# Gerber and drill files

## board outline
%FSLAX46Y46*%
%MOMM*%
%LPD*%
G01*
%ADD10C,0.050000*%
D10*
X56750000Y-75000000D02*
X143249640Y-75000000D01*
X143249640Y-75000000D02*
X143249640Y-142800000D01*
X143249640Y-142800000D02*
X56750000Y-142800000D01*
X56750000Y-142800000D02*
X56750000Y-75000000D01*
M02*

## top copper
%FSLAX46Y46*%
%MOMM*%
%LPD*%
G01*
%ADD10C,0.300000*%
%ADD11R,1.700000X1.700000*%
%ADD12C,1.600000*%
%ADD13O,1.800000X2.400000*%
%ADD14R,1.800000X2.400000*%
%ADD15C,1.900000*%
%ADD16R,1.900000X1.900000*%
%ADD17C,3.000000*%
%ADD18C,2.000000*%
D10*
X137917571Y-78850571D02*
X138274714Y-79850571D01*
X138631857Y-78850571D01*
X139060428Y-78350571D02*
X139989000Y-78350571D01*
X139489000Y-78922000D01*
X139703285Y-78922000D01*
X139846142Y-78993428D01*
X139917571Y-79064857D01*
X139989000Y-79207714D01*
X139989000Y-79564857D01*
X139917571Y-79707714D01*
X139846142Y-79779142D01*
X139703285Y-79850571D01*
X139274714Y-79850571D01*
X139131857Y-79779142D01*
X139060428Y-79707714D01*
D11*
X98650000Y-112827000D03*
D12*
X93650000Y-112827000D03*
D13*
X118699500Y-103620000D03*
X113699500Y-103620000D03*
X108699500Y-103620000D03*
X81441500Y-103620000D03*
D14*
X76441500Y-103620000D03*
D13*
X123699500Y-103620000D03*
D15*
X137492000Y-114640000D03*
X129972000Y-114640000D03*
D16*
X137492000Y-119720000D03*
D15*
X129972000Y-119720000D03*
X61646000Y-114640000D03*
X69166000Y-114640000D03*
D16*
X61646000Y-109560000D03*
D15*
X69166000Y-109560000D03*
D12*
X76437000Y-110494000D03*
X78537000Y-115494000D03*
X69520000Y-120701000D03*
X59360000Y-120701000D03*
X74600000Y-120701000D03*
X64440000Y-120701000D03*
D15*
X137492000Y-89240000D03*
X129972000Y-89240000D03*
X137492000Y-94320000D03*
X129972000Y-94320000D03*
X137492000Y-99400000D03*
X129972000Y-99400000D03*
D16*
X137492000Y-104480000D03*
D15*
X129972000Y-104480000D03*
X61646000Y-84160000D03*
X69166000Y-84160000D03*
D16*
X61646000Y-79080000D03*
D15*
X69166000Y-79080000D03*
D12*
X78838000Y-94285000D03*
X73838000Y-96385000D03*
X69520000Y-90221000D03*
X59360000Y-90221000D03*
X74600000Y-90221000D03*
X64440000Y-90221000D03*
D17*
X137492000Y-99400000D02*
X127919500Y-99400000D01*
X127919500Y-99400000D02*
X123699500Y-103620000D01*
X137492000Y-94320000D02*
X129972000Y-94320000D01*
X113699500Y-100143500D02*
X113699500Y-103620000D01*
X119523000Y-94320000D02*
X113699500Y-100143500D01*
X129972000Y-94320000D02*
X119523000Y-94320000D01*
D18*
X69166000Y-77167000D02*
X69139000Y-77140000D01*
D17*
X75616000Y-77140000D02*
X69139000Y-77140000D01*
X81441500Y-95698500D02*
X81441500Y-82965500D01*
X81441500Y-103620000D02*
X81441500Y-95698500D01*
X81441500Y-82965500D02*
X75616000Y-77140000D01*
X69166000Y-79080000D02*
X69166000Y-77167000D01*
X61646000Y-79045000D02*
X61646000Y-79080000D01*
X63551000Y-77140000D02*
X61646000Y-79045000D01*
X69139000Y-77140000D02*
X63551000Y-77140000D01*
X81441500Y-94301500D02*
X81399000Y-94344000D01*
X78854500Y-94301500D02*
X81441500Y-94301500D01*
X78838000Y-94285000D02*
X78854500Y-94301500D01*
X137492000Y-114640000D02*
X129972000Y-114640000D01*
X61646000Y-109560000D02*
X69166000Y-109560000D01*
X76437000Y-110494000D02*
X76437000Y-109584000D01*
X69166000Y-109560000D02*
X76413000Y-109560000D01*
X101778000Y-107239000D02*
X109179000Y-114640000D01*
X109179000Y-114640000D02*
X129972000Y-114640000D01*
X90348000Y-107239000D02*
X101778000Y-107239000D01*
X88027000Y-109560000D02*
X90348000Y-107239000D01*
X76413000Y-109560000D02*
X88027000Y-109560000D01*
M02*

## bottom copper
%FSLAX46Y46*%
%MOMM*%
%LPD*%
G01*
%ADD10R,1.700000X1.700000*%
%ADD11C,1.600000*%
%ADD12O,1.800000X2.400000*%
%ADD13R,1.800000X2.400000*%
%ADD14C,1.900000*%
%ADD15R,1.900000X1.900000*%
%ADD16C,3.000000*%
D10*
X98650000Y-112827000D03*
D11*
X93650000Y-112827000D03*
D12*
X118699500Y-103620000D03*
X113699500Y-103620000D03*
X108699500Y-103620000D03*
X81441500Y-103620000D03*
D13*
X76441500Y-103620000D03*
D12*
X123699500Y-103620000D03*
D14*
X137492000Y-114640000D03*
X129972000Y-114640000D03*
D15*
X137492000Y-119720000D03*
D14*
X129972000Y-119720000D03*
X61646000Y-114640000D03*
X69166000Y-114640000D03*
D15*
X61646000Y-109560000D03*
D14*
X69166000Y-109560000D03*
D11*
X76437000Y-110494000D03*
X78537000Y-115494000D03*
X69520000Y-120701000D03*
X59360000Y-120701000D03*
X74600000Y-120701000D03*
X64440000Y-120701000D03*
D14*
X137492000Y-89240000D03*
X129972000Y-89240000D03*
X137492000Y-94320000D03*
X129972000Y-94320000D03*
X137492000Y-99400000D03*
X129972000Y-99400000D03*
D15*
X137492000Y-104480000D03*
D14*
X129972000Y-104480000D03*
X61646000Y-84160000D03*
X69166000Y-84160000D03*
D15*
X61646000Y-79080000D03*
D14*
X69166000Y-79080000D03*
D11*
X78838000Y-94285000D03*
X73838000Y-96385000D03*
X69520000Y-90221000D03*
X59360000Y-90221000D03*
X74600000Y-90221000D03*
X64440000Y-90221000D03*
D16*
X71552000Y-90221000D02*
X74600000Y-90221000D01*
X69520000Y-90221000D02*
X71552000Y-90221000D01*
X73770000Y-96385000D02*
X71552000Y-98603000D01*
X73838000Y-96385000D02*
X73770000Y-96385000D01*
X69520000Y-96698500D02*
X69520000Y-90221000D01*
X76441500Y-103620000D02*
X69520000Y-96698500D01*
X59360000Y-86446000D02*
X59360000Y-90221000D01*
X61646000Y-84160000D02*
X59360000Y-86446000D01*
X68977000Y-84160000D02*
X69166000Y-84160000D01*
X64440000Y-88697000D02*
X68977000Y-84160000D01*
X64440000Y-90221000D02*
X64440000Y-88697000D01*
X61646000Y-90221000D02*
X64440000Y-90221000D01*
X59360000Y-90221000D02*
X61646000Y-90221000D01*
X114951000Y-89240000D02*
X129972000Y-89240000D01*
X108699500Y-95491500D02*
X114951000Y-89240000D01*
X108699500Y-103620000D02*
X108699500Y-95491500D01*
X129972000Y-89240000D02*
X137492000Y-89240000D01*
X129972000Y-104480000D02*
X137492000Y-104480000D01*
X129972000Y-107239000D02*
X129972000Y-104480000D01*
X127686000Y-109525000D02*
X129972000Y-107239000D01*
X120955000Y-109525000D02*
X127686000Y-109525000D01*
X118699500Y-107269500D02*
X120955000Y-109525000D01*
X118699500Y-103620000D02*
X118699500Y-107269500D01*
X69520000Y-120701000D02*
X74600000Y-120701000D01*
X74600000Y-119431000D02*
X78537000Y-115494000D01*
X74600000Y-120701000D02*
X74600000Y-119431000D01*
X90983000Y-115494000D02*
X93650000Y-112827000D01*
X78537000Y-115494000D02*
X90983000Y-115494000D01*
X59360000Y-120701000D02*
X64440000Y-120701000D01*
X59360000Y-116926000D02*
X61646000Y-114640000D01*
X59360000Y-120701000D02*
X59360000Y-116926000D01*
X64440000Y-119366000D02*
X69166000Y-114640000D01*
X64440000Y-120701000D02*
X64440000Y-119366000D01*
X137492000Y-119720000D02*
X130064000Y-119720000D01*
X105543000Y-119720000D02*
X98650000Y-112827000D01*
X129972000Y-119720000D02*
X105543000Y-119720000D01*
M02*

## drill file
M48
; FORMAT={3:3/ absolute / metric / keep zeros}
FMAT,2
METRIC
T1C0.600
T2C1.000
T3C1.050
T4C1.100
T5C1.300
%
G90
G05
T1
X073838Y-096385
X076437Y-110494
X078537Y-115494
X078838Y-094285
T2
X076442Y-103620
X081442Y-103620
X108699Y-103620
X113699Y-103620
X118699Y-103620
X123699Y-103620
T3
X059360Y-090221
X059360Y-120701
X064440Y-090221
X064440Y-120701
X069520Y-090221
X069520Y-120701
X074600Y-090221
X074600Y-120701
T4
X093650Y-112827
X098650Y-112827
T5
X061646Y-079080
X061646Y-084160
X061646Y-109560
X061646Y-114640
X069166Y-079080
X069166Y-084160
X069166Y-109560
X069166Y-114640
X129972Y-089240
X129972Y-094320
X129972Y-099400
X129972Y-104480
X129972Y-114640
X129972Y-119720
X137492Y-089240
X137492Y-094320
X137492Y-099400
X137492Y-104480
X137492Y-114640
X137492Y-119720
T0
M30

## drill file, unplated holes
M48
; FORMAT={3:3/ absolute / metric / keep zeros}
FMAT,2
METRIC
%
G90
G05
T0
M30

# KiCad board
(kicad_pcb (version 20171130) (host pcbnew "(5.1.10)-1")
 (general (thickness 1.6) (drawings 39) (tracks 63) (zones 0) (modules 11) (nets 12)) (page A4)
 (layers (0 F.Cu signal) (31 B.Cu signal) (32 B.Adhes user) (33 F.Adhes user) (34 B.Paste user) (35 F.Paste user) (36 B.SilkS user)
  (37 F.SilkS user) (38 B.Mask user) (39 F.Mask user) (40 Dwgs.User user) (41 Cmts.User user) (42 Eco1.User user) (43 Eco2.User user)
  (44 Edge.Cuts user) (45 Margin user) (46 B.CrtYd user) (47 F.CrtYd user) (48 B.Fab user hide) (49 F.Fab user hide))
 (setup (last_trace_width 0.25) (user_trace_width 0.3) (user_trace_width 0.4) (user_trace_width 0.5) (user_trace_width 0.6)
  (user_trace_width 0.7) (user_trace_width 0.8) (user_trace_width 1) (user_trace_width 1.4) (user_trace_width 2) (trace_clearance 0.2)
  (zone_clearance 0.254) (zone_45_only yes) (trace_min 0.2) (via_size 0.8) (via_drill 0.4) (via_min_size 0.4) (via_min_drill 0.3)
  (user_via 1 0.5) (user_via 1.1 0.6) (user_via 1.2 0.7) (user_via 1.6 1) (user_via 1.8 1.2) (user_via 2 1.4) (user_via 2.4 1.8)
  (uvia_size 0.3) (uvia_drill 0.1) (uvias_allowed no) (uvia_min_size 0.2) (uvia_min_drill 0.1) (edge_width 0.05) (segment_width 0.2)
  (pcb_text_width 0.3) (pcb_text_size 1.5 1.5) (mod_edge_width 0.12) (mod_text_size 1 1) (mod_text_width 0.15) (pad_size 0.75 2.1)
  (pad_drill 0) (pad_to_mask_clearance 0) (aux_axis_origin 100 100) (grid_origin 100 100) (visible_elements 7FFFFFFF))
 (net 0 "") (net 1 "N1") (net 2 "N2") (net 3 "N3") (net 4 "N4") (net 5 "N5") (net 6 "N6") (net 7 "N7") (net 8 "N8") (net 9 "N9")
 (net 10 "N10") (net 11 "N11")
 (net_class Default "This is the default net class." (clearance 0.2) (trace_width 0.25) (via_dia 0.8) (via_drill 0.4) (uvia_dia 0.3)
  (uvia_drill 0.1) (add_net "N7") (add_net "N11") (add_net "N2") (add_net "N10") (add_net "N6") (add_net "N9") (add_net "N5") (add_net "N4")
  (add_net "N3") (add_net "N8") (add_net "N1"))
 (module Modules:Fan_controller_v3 (layer F.Cu) (at 100 120.477 180)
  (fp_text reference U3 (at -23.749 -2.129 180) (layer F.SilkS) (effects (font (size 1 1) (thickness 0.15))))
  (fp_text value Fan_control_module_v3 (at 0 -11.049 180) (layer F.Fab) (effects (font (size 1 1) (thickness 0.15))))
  (pad 1 thru_hole rect (at 1.35 7.65) (size 1.7 1.7) (drill 1.1) (layers *.Cu *.Mask) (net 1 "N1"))
  (pad 2 thru_hole circle (at 6.35 7.65) (size 1.6 1.6) (drill 1.1) (layers *.Cu *.Mask) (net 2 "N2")))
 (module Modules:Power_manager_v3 (layer F.Cu) (at 100 96)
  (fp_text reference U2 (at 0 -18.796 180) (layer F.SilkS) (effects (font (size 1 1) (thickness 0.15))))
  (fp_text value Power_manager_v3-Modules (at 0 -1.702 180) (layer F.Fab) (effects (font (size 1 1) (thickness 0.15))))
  (pad 5 thru_hole oval (at 18.6995 7.62 180) (size 1.8 2.4) (drill 1) (layers *.Cu *.Mask) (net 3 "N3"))
  (pad 4 thru_hole oval (at 13.6995 7.62 180) (size 1.8 2.4) (drill 1) (layers *.Cu *.Mask) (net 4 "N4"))
  (pad 3 thru_hole oval (at 8.6995 7.62 180) (size 1.8 2.4) (drill 1) (layers *.Cu *.Mask) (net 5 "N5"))
  (pad 2 thru_hole oval (at -18.5585 7.62 180) (size 1.8 2.4) (drill 1) (layers *.Cu *.Mask) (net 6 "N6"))
  (pad 1 thru_hole rect (at -23.5585 7.62 180) (size 1.8 2.4) (drill 1) (layers *.Cu *.Mask) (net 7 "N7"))
  (pad 6 thru_hole oval (at 23.6995 7.62 180) (size 1.8 2.4) (drill 1) (layers *.Cu *.Mask) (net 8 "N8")))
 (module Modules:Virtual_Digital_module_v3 (layer F.Cu) (at 100 100)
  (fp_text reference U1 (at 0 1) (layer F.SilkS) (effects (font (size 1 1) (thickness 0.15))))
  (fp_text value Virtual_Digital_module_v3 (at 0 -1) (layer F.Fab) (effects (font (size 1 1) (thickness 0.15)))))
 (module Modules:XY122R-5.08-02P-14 (layer F.Cu) (at 137.542 119.72 90)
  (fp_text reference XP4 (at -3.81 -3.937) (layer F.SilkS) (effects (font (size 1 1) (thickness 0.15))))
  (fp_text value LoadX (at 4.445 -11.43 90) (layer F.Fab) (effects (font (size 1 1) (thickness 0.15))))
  (pad 2 thru_hole circle (at 5.08 -0.05 90) (size 1.9 1.9) (drill 1.3) (layers *.Cu *.Mask) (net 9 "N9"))
  (pad 2 thru_hole circle (at 5.08 -7.57 90) (size 1.9 1.9) (drill 1.3) (layers *.Cu *.Mask) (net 9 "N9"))
  (pad 1 thru_hole rect (at 0 -0.05 90) (size 1.9 1.9) (drill 1.3) (layers *.Cu *.Mask) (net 1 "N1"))
  (pad 1 thru_hole circle (at 0 -7.57 90) (size 1.9 1.9) (drill 1.3) (layers *.Cu *.Mask) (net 1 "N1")))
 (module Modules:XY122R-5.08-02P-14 (layer F.Cu) (at 61.596 109.56 270)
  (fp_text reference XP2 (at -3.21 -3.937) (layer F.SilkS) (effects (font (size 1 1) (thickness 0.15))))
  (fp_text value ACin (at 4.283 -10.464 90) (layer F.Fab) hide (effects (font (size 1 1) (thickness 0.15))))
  (pad 2 thru_hole circle (at 5.08 -0.05 270) (size 1.9 1.9) (drill 1.3) (layers *.Cu *.Mask) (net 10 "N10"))
  (pad 2 thru_hole circle (at 5.08 -7.57 270) (size 1.9 1.9) (drill 1.3) (layers *.Cu *.Mask) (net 10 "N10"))
  (pad 1 thru_hole rect (at 0 -0.05 270) (size 1.9 1.9) (drill 1.3) (layers *.Cu *.Mask) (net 9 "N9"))
  (pad 1 thru_hole circle (at 0 -7.57 270) (size 1.9 1.9) (drill 1.3) (layers *.Cu *.Mask) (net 9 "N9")))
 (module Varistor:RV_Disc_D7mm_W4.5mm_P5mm (layer B.Cu) (at 78.537 115.494 90)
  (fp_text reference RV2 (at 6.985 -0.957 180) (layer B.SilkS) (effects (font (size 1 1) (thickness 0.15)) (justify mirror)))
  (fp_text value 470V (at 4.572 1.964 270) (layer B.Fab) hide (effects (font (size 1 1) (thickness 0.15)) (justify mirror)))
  (pad 2 thru_hole circle (at 5 -2.1 90) (size 1.6 1.6) (drill 0.6) (layers *.Cu *.Mask) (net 9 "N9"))
  (pad 1 thru_hole circle (at 0 0 90) (size 1.6 1.6) (drill 0.6) (layers *.Cu *.Mask) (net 2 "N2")))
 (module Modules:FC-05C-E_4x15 (layer B.Cu) (at 74.6 120.701 180)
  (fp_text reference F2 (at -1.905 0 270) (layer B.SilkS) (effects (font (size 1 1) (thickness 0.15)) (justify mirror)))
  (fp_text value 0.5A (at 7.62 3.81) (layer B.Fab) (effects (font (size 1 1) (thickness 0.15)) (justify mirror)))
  (pad 1 thru_hole circle (at 5.08 0 180) (size 1.6 1.6) (drill 1.05) (layers *.Cu *.Mask) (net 2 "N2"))
  (pad 2 thru_hole circle (at 15.24 0 180) (size 1.6 1.6) (drill 1.05) (layers *.Cu *.Mask) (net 10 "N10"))
  (pad 1 thru_hole circle (at 0 0 180) (size 1.6 1.6) (drill 1.05) (layers *.Cu *.Mask) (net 2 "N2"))
  (pad 2 thru_hole circle (at 10.16 0 180) (size 1.6 1.6) (drill 1.05) (layers *.Cu *.Mask) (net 10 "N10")))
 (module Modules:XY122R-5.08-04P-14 (layer F.Cu) (at 137.542 104.48 90)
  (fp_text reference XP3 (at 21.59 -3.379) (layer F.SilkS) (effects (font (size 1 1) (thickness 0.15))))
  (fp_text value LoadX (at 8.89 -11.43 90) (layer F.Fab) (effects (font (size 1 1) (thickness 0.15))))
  (pad 4 thru_hole circle (at 15.24 -0.05 90) (size 1.9 1.9) (drill 1.3) (layers *.Cu *.Mask) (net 5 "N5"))
  (pad 4 thru_hole circle (at 15.24 -7.57 90) (size 1.9 1.9) (drill 1.3) (layers *.Cu *.Mask) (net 5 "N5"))
  (pad 3 thru_hole circle (at 10.16 -0.05 90) (size 1.9 1.9) (drill 1.3) (layers *.Cu *.Mask) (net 4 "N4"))
  (pad 3 thru_hole circle (at 10.16 -7.57 90) (size 1.9 1.9) (drill 1.3) (layers *.Cu *.Mask) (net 4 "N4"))
  (pad 2 thru_hole circle (at 5.08 -0.05 90) (size 1.9 1.9) (drill 1.3) (layers *.Cu *.Mask) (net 8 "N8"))
  (pad 2 thru_hole circle (at 5.08 -7.57 90) (size 1.9 1.9) (drill 1.3) (layers *.Cu *.Mask) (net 8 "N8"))
  (pad 1 thru_hole rect (at 0 -0.05 90) (size 1.9 1.9) (drill 1.3) (layers *.Cu *.Mask) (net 3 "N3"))
  (pad 1 thru_hole circle (at 0 -7.57 90) (size 1.9 1.9) (drill 1.3) (layers *.Cu *.Mask) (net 3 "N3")))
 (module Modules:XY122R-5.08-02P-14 (layer F.Cu) (at 61.596 79.08 270)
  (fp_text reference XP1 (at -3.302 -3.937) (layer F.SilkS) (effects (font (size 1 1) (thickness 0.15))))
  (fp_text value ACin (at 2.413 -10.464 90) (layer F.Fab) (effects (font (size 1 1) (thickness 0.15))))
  (pad 2 thru_hole circle (at 5.08 -0.05 270) (size 1.9 1.9) (drill 1.3) (layers *.Cu *.Mask) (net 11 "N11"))
  (pad 2 thru_hole circle (at 5.08 -7.57 270) (size 1.9 1.9) (drill 1.3) (layers *.Cu *.Mask) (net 11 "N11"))
  (pad 1 thru_hole rect (at 0 -0.05 270) (size 1.9 1.9) (drill 1.3) (layers *.Cu *.Mask) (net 6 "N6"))
  (pad 1 thru_hole circle (at 0 -7.57 270) (size 1.9 1.9) (drill 1.3) (layers *.Cu *.Mask) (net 6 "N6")))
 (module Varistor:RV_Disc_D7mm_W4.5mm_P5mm (layer B.Cu) (at 73.838 96.385)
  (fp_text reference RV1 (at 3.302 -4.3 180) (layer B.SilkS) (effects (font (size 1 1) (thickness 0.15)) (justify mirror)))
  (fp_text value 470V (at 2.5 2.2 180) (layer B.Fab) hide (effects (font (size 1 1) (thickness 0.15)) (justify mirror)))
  (pad 2 thru_hole circle (at 5 -2.1) (size 1.6 1.6) (drill 0.6) (layers *.Cu *.Mask) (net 6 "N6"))
  (pad 1 thru_hole circle (at 0 0) (size 1.6 1.6) (drill 0.6) (layers *.Cu *.Mask) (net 7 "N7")))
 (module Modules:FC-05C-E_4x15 (layer B.Cu) (at 74.6 90.221 180)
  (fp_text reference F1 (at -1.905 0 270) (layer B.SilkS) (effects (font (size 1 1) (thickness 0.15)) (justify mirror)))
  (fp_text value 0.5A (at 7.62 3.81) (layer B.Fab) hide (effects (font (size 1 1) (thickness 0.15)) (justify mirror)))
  (pad 1 thru_hole circle (at 5.08 0 180) (size 1.6 1.6) (drill 1.05) (layers *.Cu *.Mask) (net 7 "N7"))
  (pad 2 thru_hole circle (at 15.24 0 180) (size 1.6 1.6) (drill 1.05) (layers *.Cu *.Mask) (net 11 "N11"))
  (pad 1 thru_hole circle (at 0 0 180) (size 1.6 1.6) (drill 1.05) (layers *.Cu *.Mask) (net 7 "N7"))
  (pad 2 thru_hole circle (at 10.16 0 180) (size 1.6 1.6) (drill 1.05) (layers *.Cu *.Mask) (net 11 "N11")))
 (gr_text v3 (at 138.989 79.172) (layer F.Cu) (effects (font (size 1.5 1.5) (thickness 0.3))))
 (gr_line (start 56.75 75) (end 143.24964 75) (layer Edge.Cuts) (width 0.05))
 (gr_line (start 143.24964 75) (end 143.24964 142.8) (layer Edge.Cuts) (width 0.05))
 (gr_line (start 143.24964 142.8) (end 56.75 142.8) (layer Edge.Cuts) (width 0.05))
 (gr_line (start 56.75 142.8) (end 56.75 75) (layer Edge.Cuts) (width 0.05))
 (segment (start 71.552 90.221) (end 74.6 90.221) (width 3) (layer B.Cu) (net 7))
 (segment (start 69.52 90.221) (end 71.552 90.221) (width 3) (layer B.Cu) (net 7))
 (segment (start 73.77 96.385) (end 71.552 98.603) (width 3) (layer B.Cu) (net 7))
 (segment (start 73.838 96.385) (end 73.77 96.385) (width 3) (layer B.Cu) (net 7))
 (segment (start 69.52 96.6985) (end 69.52 90.221) (width 3) (layer B.Cu) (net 7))
 (segment (start 76.4415 103.62) (end 69.52 96.6985) (width 3) (layer B.Cu) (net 7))
 (segment (start 59.36 86.446) (end 59.36 90.221) (width 3) (layer B.Cu) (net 11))
 (segment (start 61.646 84.16) (end 59.36 86.446) (width 3) (layer B.Cu) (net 11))
 (segment (start 68.977 84.16) (end 69.166 84.16) (width 3) (layer B.Cu) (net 11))
 (segment (start 64.44 88.697) (end 68.977 84.16) (width 3) (layer B.Cu) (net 11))
 (segment (start 64.44 90.221) (end 64.44 88.697) (width 3) (layer B.Cu) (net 11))
 (segment (start 61.646 90.221) (end 64.44 90.221) (width 3) (layer B.Cu) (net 11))
 (segment (start 59.36 90.221) (end 61.646 90.221) (width 3) (layer B.Cu) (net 11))
 (segment (start 137.492 99.4) (end 127.9195 99.4) (width 3) (layer F.Cu) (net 8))
 (segment (start 127.9195 99.4) (end 123.6995 103.62) (width 3) (layer F.Cu) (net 8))
 (segment (start 114.951 89.24) (end 129.972 89.24) (width 3) (layer B.Cu) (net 5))
 (segment (start 108.6995 95.4915) (end 114.951 89.24) (width 3) (layer B.Cu) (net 5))
 (segment (start 108.6995 103.62) (end 108.6995 95.4915) (width 3) (layer B.Cu) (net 5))
 (segment (start 129.972 89.24) (end 137.492 89.24) (width 3) (layer B.Cu) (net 5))
 (segment (start 137.492 94.32) (end 129.972 94.32) (width 3) (layer F.Cu) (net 4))
 (segment (start 113.6995 100.1435) (end 113.6995 103.62) (width 3) (layer F.Cu) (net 4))
 (segment (start 119.523 94.32) (end 113.6995 100.1435) (width 3) (layer F.Cu) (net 4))
 (segment (start 129.972 94.32) (end 119.523 94.32) (width 3) (layer F.Cu) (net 4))
 (segment (start 129.972 104.48) (end 137.492 104.48) (width 3) (layer B.Cu) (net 3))
 (segment (start 129.972 107.239) (end 129.972 104.48) (width 3) (layer B.Cu) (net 3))
 (segment (start 127.686 109.525) (end 129.972 107.239) (width 3) (layer B.Cu) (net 3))
 (segment (start 120.955 109.525) (end 127.686 109.525) (width 3) (layer B.Cu) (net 3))
 (segment (start 118.6995 107.2695) (end 120.955 109.525) (width 3) (layer B.Cu) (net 3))
 (segment (start 118.6995 103.62) (end 118.6995 107.2695) (width 3) (layer B.Cu) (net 3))
 (segment (start 69.166 77.167) (end 69.139 77.14) (width 2) (layer F.Cu) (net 6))
 (segment (start 75.616 77.14) (end 69.139 77.14) (width 3) (layer F.Cu) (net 6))
 (segment (start 81.4415 95.6985) (end 81.4415 82.9655) (width 3) (layer F.Cu) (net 6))
 (segment (start 81.4415 103.62) (end 81.4415 95.6985) (width 3) (layer F.Cu) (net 6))
 (segment (start 81.4415 82.9655) (end 75.616 77.14) (width 3) (layer F.Cu) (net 6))
 (segment (start 69.166 79.08) (end 69.166 77.167) (width 3) (layer F.Cu) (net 6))
 (segment (start 61.646 79.045) (end 61.646 79.08) (width 3) (layer F.Cu) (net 6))
 (segment (start 63.551 77.14) (end 61.646 79.045) (width 3) (layer F.Cu) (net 6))
 (segment (start 69.139 77.14) (end 63.551 77.14) (width 3) (layer F.Cu) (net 6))
 (segment (start 81.4415 94.3015) (end 81.399 94.344) (width 3) (layer F.Cu) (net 6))
 (segment (start 78.8545 94.3015) (end 81.4415 94.3015) (width 3) (layer F.Cu) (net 6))
 (segment (start 78.838 94.285) (end 78.8545 94.3015) (width 3) (layer F.Cu) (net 6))
 (segment (start 69.52 120.701) (end 74.6 120.701) (width 3) (layer B.Cu) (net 2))
 (segment (start 74.6 119.431) (end 78.537 115.494) (width 3) (layer B.Cu) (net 2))
 (segment (start 74.6 120.701) (end 74.6 119.431) (width 3) (layer B.Cu) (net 2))
 (segment (start 90.983 115.494) (end 93.65 112.827) (width 3) (layer B.Cu) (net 2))
 (segment (start 78.537 115.494) (end 90.983 115.494) (width 3) (layer B.Cu) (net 2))
 (segment (start 59.36 120.701) (end 64.44 120.701) (width 3) (layer B.Cu) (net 10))
 (segment (start 59.36 116.926) (end 61.646 114.64) (width 3) (layer B.Cu) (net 10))
 (segment (start 59.36 120.701) (end 59.36 116.926) (width 3) (layer B.Cu) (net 10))
 (segment (start 64.44 119.366) (end 69.166 114.64) (width 3) (layer B.Cu) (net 10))
 (segment (start 64.44 120.701) (end 64.44 119.366) (width 3) (layer B.Cu) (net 10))
 (segment (start 137.492 114.64) (end 129.972 114.64) (width 3) (layer F.Cu) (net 9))
 (segment (start 61.646 109.56) (end 69.166 109.56) (width 3) (layer F.Cu) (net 9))
 (segment (start 76.437 110.494) (end 76.437 109.584) (width 3) (layer F.Cu) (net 9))
 (segment (start 69.166 109.56) (end 76.413 109.56) (width 3) (layer F.Cu) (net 9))
 (segment (start 101.778 107.239) (end 109.179 114.64) (width 3) (layer F.Cu) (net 9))
 (segment (start 109.179 114.64) (end 129.972 114.64) (width 3) (layer F.Cu) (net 9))
 (segment (start 90.348 107.239) (end 101.778 107.239) (width 3) (layer F.Cu) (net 9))
 (segment (start 88.027 109.56) (end 90.348 107.239) (width 3) (layer F.Cu) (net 9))
 (segment (start 76.413 109.56) (end 88.027 109.56) (width 3) (layer F.Cu) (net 9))
 (segment (start 137.492 119.72) (end 130.064 119.72) (width 3) (layer B.Cu) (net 1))
 (segment (start 105.543 119.72) (end 98.65 112.827) (width 3) (layer B.Cu) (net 1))
 (segment (start 129.972 119.72) (end 105.543 119.72) (width 3) (layer B.Cu) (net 1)))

